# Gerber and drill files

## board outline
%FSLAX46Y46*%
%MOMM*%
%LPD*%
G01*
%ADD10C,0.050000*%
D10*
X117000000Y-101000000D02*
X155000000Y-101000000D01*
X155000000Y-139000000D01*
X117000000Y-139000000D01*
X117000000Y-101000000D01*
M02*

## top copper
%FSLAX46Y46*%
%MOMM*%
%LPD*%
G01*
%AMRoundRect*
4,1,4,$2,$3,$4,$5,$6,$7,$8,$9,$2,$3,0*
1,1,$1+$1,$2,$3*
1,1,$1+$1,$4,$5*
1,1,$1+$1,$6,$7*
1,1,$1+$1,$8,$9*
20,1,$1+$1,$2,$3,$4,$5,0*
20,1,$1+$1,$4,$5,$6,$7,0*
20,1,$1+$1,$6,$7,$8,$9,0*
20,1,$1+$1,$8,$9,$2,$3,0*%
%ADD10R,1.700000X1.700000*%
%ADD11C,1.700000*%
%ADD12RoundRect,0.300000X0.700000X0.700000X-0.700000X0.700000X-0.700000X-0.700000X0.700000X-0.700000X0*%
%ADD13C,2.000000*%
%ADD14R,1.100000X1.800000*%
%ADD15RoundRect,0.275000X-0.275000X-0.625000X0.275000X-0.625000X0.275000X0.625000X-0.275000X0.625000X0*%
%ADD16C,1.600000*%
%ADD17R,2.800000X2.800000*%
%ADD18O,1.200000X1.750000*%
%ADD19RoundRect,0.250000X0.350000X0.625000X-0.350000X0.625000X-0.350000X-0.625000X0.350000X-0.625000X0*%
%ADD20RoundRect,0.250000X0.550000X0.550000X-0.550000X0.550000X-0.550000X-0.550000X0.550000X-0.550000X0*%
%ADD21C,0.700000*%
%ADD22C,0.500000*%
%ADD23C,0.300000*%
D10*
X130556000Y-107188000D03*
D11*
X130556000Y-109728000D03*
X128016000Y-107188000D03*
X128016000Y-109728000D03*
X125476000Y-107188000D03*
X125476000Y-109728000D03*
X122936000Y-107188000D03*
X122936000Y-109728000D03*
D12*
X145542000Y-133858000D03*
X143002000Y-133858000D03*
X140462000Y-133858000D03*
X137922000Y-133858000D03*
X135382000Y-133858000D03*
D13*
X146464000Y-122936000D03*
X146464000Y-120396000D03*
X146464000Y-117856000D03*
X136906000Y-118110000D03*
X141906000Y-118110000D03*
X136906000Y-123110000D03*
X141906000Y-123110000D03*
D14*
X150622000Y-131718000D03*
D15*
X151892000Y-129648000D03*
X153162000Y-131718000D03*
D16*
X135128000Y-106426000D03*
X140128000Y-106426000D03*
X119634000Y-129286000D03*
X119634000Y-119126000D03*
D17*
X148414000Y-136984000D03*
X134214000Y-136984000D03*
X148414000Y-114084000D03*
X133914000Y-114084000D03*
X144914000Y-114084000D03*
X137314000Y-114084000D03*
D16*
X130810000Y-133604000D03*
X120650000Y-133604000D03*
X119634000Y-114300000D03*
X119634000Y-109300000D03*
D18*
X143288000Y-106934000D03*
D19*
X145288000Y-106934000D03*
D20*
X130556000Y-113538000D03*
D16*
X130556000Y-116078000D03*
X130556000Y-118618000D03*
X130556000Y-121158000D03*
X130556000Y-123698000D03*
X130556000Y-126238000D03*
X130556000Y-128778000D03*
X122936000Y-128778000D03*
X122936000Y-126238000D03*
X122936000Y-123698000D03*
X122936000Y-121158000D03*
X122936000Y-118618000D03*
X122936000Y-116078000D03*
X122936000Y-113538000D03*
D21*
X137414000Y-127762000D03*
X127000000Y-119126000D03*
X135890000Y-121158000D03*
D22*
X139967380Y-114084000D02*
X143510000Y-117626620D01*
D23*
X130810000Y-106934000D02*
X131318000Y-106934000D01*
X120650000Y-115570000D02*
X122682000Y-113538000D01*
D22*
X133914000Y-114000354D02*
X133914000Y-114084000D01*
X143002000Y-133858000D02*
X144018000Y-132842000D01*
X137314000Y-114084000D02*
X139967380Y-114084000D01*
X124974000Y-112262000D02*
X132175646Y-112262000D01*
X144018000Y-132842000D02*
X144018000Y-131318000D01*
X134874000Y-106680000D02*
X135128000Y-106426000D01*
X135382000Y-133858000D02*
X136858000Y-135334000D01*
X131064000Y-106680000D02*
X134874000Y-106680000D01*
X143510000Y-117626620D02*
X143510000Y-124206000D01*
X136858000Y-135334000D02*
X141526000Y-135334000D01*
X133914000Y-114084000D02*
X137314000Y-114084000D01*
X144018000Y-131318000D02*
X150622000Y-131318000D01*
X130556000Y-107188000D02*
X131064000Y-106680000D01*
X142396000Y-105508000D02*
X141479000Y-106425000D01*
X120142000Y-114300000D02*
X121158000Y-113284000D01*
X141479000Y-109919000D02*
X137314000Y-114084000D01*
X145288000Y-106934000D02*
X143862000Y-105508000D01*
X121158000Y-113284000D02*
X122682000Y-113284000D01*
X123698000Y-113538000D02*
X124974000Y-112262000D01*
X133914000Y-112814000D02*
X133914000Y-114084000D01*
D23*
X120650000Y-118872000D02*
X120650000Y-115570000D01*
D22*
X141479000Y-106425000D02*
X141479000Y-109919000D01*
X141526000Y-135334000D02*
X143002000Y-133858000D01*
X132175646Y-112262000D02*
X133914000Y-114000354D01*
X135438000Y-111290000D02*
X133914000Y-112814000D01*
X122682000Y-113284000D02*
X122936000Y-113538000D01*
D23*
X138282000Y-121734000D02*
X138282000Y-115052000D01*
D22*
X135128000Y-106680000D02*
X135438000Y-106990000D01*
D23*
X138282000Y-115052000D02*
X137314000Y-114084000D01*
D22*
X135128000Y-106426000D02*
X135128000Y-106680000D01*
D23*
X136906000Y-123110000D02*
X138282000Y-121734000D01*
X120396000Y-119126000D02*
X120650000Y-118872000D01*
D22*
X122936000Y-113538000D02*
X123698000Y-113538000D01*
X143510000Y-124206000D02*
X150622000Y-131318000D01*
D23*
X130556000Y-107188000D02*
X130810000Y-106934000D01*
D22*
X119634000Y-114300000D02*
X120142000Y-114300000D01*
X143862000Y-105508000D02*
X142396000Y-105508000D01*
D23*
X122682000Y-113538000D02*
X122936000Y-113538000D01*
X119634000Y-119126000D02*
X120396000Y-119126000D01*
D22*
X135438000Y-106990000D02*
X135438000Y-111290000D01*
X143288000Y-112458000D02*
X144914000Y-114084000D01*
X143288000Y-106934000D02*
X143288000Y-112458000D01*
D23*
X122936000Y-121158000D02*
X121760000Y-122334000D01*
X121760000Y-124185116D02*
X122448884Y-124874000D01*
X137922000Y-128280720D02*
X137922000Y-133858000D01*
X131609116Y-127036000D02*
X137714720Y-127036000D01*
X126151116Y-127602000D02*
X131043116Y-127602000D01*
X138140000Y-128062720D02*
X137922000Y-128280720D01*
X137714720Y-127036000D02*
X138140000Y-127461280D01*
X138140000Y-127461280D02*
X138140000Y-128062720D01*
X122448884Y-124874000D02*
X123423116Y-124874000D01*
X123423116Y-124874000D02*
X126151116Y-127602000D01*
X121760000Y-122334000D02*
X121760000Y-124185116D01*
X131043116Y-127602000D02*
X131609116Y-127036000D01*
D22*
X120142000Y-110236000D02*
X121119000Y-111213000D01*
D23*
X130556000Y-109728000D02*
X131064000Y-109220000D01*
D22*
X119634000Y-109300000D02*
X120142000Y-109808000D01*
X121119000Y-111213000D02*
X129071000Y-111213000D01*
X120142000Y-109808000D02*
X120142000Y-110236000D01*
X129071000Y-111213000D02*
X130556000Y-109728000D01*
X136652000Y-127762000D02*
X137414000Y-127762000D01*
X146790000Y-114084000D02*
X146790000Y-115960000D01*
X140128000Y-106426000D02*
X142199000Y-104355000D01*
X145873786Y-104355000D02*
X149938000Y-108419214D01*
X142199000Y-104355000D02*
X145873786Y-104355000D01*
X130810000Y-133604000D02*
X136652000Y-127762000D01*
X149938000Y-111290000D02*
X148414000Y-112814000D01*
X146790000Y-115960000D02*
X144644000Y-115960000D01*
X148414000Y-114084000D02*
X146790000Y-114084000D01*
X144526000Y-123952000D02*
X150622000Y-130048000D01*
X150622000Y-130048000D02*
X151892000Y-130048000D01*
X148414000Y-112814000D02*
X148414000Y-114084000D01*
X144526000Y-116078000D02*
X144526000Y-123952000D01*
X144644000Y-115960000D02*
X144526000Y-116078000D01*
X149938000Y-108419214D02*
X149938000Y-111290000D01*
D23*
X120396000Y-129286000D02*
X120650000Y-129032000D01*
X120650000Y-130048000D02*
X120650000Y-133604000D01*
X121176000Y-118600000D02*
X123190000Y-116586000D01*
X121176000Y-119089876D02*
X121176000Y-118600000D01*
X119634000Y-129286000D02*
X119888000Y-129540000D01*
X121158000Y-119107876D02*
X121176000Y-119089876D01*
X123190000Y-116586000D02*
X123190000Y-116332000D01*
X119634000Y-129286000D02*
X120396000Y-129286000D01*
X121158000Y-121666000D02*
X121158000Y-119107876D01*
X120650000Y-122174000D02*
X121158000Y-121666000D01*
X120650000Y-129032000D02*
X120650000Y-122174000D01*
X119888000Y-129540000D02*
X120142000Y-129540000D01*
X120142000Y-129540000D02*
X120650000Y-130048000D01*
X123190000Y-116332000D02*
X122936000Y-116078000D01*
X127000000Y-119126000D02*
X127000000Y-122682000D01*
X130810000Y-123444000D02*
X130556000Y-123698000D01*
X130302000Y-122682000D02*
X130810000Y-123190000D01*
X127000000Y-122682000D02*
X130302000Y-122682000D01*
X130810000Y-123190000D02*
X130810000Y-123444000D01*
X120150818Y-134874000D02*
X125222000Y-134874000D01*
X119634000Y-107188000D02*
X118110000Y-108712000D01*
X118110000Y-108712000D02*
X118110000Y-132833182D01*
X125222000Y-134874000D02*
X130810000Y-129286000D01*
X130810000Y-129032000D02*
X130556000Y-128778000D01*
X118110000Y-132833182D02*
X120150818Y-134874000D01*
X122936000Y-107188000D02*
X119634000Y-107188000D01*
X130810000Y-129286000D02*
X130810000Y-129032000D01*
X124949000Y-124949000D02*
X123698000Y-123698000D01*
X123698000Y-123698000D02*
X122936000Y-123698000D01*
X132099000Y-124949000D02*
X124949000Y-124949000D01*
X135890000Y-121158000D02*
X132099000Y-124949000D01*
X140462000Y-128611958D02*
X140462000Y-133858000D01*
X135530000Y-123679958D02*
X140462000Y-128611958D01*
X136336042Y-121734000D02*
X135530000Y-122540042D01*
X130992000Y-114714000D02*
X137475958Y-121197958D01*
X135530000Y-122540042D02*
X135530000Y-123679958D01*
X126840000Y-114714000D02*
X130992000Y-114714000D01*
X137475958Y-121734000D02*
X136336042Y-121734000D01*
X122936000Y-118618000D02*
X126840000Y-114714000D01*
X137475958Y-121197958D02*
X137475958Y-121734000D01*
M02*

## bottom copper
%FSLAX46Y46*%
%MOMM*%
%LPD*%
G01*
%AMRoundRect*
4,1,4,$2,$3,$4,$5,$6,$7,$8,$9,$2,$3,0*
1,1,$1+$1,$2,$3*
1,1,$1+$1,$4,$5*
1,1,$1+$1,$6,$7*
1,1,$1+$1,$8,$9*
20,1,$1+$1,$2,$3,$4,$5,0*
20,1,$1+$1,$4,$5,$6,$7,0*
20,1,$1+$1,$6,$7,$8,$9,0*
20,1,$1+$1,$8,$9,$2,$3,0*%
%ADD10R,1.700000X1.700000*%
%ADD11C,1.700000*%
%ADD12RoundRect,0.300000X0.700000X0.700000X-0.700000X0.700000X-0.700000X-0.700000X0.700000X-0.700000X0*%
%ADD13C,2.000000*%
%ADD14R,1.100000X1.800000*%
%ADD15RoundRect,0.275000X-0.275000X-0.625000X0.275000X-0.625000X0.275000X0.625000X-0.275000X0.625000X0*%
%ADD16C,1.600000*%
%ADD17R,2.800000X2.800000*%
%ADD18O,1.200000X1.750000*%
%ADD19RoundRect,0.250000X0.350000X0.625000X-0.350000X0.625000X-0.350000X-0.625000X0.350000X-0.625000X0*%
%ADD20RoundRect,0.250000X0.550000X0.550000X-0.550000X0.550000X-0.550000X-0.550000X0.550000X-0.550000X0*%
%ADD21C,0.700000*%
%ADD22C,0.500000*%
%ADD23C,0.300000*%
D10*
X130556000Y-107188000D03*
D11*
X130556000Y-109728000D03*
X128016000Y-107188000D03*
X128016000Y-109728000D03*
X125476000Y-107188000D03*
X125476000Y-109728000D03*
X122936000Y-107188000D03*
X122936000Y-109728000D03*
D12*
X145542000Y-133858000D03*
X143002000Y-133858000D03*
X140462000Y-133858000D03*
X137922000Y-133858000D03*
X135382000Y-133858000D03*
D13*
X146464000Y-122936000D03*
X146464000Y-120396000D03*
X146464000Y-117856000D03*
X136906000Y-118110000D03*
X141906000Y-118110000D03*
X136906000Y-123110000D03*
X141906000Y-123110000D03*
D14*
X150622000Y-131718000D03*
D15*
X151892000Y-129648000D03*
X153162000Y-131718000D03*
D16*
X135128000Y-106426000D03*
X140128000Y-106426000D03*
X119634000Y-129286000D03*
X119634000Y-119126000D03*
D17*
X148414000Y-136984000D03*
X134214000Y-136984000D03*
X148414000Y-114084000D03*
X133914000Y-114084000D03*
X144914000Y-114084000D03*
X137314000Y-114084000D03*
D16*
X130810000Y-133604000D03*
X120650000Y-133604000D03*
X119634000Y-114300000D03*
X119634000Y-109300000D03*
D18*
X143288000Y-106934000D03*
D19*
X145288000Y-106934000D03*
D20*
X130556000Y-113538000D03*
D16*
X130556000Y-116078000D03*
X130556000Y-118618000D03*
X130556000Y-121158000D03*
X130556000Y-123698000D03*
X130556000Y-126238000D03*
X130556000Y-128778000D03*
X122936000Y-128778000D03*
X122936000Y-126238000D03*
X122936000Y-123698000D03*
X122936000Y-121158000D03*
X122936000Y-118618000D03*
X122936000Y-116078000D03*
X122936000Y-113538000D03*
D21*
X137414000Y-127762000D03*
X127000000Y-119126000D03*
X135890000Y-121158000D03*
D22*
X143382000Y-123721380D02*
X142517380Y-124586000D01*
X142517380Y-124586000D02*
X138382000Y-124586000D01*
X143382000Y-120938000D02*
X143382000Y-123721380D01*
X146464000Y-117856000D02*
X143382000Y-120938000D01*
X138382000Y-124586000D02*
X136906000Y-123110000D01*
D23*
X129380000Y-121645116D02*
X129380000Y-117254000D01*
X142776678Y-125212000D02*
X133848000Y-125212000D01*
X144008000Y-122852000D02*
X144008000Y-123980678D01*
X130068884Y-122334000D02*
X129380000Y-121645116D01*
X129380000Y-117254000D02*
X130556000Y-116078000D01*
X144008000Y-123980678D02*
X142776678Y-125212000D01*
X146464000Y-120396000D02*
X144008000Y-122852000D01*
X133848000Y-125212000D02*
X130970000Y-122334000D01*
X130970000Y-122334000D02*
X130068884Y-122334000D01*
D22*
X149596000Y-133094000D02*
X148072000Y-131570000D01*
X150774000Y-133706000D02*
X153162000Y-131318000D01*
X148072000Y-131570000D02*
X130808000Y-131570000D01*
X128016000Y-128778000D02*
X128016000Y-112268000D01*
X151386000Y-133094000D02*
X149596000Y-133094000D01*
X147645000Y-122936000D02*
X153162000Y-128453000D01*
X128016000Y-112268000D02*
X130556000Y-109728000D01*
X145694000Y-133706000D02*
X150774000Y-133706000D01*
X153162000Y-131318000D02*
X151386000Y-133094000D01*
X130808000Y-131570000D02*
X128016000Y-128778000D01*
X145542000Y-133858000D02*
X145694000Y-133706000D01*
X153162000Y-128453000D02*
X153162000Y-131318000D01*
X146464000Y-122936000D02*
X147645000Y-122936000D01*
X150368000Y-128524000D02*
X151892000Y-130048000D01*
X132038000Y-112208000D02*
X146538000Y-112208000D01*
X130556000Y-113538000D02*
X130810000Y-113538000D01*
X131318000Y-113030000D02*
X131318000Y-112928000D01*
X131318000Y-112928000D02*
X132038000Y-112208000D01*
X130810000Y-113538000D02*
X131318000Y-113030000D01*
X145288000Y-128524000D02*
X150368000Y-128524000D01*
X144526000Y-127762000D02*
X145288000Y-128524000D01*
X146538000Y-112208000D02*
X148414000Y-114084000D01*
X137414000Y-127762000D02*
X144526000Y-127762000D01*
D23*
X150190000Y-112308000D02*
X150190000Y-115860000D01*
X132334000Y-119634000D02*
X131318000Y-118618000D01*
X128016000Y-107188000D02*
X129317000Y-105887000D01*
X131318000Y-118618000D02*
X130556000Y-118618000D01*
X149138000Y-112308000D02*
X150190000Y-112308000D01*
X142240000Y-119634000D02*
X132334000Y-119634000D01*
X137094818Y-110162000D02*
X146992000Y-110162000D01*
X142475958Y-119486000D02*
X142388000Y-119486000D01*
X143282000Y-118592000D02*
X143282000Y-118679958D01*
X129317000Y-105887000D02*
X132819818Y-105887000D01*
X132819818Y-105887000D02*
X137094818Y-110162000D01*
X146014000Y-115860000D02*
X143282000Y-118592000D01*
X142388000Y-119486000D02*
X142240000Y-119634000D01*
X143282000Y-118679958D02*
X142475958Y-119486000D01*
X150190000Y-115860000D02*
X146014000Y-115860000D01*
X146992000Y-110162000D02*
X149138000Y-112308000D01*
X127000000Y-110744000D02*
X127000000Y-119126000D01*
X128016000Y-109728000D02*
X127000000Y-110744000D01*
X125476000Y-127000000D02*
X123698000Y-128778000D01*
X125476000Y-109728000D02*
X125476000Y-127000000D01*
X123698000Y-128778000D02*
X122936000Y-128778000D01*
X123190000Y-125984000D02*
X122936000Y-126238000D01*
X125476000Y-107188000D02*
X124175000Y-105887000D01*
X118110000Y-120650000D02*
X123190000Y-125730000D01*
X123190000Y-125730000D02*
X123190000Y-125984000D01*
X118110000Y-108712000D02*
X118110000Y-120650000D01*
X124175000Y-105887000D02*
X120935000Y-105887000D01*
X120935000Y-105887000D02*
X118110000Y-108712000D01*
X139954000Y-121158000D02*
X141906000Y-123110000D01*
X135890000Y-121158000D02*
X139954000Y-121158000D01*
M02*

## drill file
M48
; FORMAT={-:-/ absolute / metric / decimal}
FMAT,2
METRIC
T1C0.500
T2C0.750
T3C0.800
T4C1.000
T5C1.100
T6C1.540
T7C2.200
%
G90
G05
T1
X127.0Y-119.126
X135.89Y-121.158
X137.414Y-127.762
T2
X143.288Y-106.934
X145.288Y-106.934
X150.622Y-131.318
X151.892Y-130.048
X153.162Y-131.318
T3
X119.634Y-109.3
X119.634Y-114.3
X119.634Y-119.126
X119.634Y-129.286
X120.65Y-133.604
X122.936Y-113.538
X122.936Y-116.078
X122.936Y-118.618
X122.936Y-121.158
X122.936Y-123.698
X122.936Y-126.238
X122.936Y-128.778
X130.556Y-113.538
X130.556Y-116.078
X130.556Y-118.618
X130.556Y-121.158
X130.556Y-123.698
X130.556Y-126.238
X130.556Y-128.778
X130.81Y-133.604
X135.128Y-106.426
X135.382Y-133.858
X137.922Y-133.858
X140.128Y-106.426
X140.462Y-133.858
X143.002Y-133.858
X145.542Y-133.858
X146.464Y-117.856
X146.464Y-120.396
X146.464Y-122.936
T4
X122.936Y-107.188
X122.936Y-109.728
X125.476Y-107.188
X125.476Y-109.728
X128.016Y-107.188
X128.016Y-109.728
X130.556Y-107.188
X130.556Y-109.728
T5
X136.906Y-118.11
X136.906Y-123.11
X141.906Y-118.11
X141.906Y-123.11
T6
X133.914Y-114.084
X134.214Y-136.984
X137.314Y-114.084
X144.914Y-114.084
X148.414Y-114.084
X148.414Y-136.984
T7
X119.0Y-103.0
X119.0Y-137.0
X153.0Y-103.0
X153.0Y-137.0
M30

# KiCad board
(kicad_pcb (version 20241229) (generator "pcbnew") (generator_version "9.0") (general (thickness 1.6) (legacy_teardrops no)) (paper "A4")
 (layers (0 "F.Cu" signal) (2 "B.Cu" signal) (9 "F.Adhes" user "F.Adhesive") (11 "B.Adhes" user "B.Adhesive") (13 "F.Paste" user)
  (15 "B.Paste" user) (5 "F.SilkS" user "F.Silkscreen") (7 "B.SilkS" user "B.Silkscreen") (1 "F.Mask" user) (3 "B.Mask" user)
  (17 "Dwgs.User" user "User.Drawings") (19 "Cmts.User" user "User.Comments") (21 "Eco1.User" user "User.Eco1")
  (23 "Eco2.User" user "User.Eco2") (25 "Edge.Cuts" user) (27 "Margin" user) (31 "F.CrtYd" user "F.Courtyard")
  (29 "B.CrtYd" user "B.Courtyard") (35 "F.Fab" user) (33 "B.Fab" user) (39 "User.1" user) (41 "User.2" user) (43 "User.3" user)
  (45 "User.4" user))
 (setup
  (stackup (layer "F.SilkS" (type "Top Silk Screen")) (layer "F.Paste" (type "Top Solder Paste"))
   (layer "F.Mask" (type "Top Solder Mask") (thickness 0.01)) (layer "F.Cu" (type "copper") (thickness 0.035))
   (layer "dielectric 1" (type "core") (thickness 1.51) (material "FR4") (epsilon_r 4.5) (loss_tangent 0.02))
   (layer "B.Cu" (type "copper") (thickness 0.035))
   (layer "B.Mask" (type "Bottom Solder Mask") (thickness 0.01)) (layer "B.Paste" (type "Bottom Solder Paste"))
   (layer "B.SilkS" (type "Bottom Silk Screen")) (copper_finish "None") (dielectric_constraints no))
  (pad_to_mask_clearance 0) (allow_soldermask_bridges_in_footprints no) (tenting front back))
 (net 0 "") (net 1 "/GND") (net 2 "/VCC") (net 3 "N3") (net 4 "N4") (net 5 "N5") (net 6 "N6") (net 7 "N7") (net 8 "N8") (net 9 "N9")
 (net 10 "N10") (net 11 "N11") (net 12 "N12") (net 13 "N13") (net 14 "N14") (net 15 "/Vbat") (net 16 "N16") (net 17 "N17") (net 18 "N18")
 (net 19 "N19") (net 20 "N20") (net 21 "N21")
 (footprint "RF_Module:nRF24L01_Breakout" (layer "F.Cu") (at 130.556 107.188 -90)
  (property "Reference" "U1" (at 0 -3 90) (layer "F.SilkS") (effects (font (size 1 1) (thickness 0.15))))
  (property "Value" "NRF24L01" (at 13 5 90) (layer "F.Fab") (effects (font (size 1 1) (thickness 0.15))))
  (pad "1" thru_hole rect (at 0 0 270) (size 1.7 1.7) (drill 1) (layers "*.Cu" "*.Mask") (remove_unused_layers no) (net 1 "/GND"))
  (pad "2" thru_hole circle (at 2.54 0 270) (size 1.7 1.7) (drill 1) (layers "*.Cu" "*.Mask") (remove_unused_layers no) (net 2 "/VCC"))
  (pad "3" thru_hole circle (at 0 2.54 270) (size 1.7 1.7) (drill 1) (layers "*.Cu" "*.Mask") (remove_unused_layers no) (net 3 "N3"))
  (pad "4" thru_hole circle (at 2.54 2.54 270) (size 1.7 1.7) (drill 1) (layers "*.Cu" "*.Mask") (remove_unused_layers no) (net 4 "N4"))
  (pad "5" thru_hole circle (at 0 5.08 270) (size 1.7 1.7) (drill 1) (layers "*.Cu" "*.Mask") (remove_unused_layers no) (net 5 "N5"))
  (pad "6" thru_hole circle (at 2.54 5.08 270) (size 1.7 1.7) (drill 1) (layers "*.Cu" "*.Mask") (remove_unused_layers no) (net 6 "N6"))
  (pad "7" thru_hole circle (at 0 7.62 270) (size 1.7 1.7) (drill 1) (layers "*.Cu" "*.Mask") (remove_unused_layers no) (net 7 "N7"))
  (pad "8" thru_hole circle (at 2.54 7.62 270) (size 1.7 1.7) (drill 1) (layers "*.Cu" "*.Mask") (remove_unused_layers no) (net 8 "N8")))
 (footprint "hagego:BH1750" (layer "F.Cu") (at 140.462 135.128 180)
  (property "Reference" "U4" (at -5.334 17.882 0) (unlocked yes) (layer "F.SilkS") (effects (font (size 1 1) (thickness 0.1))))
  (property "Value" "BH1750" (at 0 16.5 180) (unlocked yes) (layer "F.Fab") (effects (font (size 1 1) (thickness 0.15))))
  (pad "1" thru_hole roundrect (at -5.08 1.27 180) (size 2 2) (drill 0.8) (layers "*.Cu" "*.Mask") (remove_unused_layers no)
   (roundrect_rratio 0.15) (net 2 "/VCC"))
  (pad "2" thru_hole roundrect (at -2.54 1.27 180) (size 2 2) (drill 0.8) (layers "*.Cu" "*.Mask") (remove_unused_layers no)
   (roundrect_rratio 0.15) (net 1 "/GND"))
  (pad "3" thru_hole roundrect (at 0 1.27 180) (size 2 2) (drill 0.8) (layers "*.Cu" "*.Mask") (remove_unused_layers no)
   (roundrect_rratio 0.15) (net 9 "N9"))
  (pad "4" thru_hole roundrect (at 2.54 1.27 180) (size 2 2) (drill 0.8) (layers "*.Cu" "*.Mask") (remove_unused_layers no)
   (roundrect_rratio 0.15) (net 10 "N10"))
  (pad "5" thru_hole roundrect (at 5.08 1.27 180) (size 2 2) (drill 0.8) (layers "*.Cu" "*.Mask") (remove_unused_layers no)
   (roundrect_rratio 0.15) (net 1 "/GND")))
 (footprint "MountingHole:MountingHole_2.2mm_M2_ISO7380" (layer "F.Cu") (at 153 137)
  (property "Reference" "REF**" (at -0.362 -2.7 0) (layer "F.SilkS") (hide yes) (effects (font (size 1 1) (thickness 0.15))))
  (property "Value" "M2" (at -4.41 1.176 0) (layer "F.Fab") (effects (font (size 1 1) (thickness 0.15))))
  (pad "" np_thru_hole circle (at 0 0) (size 2.2 2.2) (drill 2.2) (layers "*.Cu" "*.Mask")))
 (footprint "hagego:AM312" (layer "F.Cu") (at 148.336 120.396 90)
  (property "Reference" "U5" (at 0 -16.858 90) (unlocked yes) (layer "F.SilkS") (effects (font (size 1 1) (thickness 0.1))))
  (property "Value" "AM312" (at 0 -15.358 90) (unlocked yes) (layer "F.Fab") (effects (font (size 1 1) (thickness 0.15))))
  (pad "1" thru_hole circle (at -2.54 -1.872 90) (size 2 2) (drill 0.8) (layers "*.Cu" "*.Mask") (remove_unused_layers no) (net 2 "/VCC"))
  (pad "2" thru_hole circle (at 0 -1.872 90) (size 2 2) (drill 0.8) (layers "*.Cu" "*.Mask") (remove_unused_layers no) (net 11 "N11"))
  (pad "3" thru_hole circle (at 2.54 -1.872 90) (size 2 2) (drill 0.8) (layers "*.Cu" "*.Mask") (remove_unused_layers no) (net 1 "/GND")))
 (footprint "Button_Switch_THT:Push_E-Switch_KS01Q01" (layer "F.Cu") (at 136.906 118.11)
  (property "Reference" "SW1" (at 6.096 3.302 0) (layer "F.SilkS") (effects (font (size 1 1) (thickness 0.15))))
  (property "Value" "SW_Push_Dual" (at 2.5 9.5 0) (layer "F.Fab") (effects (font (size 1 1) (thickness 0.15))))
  (pad "1" thru_hole circle (at 0 0) (size 2 2) (drill 1.1) (layers "*.Cu" "*.Mask") (remove_unused_layers no) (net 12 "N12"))
  (pad "2" thru_hole circle (at 5 0) (size 2 2) (drill 1.1) (layers "*.Cu" "*.Mask") (remove_unused_layers no) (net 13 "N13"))
  (pad "3" thru_hole circle (at 0 5) (size 2 2) (drill 1.1) (layers "*.Cu" "*.Mask") (remove_unused_layers no) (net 1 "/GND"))
  (pad "4" thru_hole circle (at 5 5) (size 2 2) (drill 1.1) (layers "*.Cu" "*.Mask") (remove_unused_layers no) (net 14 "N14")))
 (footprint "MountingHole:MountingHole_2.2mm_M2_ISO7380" (layer "F.Cu") (at 119 137)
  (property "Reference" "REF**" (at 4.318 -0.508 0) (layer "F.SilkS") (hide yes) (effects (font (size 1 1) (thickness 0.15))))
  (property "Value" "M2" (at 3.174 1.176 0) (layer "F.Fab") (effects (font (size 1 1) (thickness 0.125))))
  (pad "" np_thru_hole circle (at 0 0) (size 2.2 2.2) (drill 2.2) (layers "*.Cu" "*.Mask")))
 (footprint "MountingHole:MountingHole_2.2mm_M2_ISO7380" (layer "F.Cu") (at 119 103)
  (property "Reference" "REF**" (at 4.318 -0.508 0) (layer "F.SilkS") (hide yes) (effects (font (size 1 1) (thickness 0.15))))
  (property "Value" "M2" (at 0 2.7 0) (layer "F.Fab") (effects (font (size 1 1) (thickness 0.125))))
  (pad "" np_thru_hole circle (at 0 0) (size 2.2 2.2) (drill 2.2) (layers "*.Cu" "*.Mask")))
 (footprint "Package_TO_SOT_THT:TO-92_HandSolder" (layer "F.Cu") (at 150.622 131.318)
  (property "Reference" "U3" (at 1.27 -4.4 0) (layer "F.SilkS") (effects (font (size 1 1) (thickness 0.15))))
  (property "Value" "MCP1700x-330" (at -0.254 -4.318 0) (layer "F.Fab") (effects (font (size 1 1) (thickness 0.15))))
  (pad "1" thru_hole rect (at 0 0) (size 1.1 1.8) (drill 0.75 (offset 0 0.4)) (layers "*.Cu" "*.Mask") (remove_unused_layers no)
   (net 1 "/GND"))
  (pad "2" thru_hole roundrect (at 1.27 -1.27) (size 1.1 1.8) (drill 0.75 (offset 0 -0.4)) (layers "*.Cu" "*.Mask")
   (remove_unused_layers no) (roundrect_rratio 0.25) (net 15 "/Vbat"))
  (pad "3" thru_hole roundrect (at 2.54 0) (size 1.1 1.8) (drill 0.75 (offset 0 0.4)) (layers "*.Cu" "*.Mask") (remove_unused_layers no)
   (roundrect_rratio 0.25) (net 2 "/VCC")))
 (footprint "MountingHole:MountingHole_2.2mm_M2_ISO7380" (layer "F.Cu") (at 153 103)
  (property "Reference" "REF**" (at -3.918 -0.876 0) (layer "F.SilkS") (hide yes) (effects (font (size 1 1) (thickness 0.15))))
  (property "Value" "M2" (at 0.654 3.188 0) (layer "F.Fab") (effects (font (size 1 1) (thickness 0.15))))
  (pad "" np_thru_hole circle (at 0 0) (size 2.2 2.2) (drill 2.2) (layers "*.Cu" "*.Mask")))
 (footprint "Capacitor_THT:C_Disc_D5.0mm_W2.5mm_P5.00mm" (layer "F.Cu") (at 135.128 106.426)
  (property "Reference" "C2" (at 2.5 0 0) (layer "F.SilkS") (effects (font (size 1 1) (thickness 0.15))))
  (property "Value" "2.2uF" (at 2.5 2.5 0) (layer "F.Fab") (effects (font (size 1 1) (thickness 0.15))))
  (pad "1" thru_hole circle (at 0 0) (size 1.6 1.6) (drill 0.8) (layers "*.Cu" "*.Mask") (remove_unused_layers no) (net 1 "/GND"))
  (pad "2" thru_hole circle (at 5 0) (size 1.6 1.6) (drill 0.8) (layers "*.Cu" "*.Mask") (remove_unused_layers no) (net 15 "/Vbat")))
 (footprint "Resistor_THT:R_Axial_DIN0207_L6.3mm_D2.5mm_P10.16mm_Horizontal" (layer "B.Cu") (at 119.634 129.286 90)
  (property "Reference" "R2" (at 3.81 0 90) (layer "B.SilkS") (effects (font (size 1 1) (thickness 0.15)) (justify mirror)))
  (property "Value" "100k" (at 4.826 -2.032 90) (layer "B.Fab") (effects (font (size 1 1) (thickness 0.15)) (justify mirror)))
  (pad "1" thru_hole circle (at 0 0 90) (size 1.6 1.6) (drill 0.8) (layers "*.Cu" "*.Mask") (remove_unused_layers no) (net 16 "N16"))
  (pad "2" thru_hole circle (at 10.16 0 90) (size 1.6 1.6) (drill 0.8) (layers "*.Cu" "*.Mask") (remove_unused_layers no) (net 1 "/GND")))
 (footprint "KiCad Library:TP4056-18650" (layer "B.Cu") (at 150.114 138.684 90)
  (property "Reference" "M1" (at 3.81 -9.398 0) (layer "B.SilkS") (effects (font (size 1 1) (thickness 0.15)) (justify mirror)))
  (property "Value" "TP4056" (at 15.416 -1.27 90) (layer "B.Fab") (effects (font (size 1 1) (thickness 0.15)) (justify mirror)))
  (pad "1" thru_hole rect (at 1.7 -1.7 90) (size 2.8 2.8) (drill 1.54) (layers "*.Cu" "*.Mask") (remove_unused_layers no) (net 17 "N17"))
  (pad "2" thru_hole rect (at 1.7 -15.9 90) (size 2.8 2.8) (drill 1.54) (layers "*.Cu" "*.Mask") (remove_unused_layers no) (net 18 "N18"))
  (pad "3" thru_hole rect (at 24.6 -1.7 90) (size 2.8 2.8) (drill 1.54) (layers "*.Cu" "*.Mask") (remove_unused_layers no) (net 15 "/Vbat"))
  (pad "4" thru_hole rect (at 24.6 -16.2 90) (size 2.8 2.8) (drill 1.54) (layers "*.Cu" "*.Mask") (remove_unused_layers no) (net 1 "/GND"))
  (pad "5" thru_hole rect (at 24.6 -5.2 90) (size 2.8 2.8) (drill 1.54) (layers "*.Cu" "*.Mask") (remove_unused_layers no) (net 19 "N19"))
  (pad "6" thru_hole rect (at 24.6 -12.8 90) (size 2.8 2.8) (drill 1.54) (layers "*.Cu" "*.Mask") (remove_unused_layers no) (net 1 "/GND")))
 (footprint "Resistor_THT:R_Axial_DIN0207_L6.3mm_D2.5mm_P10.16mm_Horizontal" (layer "B.Cu") (at 130.81 133.604 180)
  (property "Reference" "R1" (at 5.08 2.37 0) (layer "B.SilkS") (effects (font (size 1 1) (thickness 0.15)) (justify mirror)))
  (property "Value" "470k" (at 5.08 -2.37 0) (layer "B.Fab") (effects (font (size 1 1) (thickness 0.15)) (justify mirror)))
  (pad "1" thru_hole circle (at 0 0 180) (size 1.6 1.6) (drill 0.8) (layers "*.Cu" "*.Mask") (remove_unused_layers no) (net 15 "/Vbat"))
  (pad "2" thru_hole circle (at 10.16 0 180) (size 1.6 1.6) (drill 0.8) (layers "*.Cu" "*.Mask") (remove_unused_layers no) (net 16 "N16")))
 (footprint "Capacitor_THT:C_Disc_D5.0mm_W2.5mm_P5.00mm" (layer "B.Cu") (at 119.634 114.3 90)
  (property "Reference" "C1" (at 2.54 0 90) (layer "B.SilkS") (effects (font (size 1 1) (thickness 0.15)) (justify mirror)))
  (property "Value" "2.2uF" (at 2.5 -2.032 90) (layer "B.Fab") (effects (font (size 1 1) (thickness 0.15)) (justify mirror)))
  (pad "1" thru_hole circle (at 0 0 90) (size 1.6 1.6) (drill 0.8) (layers "*.Cu" "*.Mask") (remove_unused_layers no) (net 1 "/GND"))
  (pad "2" thru_hole circle (at 5 0 90) (size 1.6 1.6) (drill 0.8) (layers "*.Cu" "*.Mask") (remove_unused_layers no) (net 2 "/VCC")))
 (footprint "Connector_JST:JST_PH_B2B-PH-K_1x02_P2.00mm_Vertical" (layer "B.Cu") (at 145.288 106.934 180)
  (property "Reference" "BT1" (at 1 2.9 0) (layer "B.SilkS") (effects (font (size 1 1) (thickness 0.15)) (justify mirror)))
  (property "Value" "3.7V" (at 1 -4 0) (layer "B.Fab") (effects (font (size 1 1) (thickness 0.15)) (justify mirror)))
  (pad "1" thru_hole oval (at 2 0 180) (size 1.2 1.75) (drill 0.75) (layers "*.Cu" "*.Mask") (remove_unused_layers no) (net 19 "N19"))
  (pad "2" thru_hole roundrect (at 0 0 180) (size 1.2 1.75) (drill 0.75) (layers "*.Cu" "*.Mask") (remove_unused_layers no)
   (roundrect_rratio 0.208333) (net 1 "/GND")))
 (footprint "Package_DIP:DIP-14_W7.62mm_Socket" (layer "B.Cu") (at 130.556 113.538 180)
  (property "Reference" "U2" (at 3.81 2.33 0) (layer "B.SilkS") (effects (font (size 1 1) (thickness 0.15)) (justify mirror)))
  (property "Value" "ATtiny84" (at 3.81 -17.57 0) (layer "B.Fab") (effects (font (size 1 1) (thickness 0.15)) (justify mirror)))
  (pad "1" thru_hole roundrect (at 0 0 180) (size 1.6 1.6) (drill 0.8) (layers "*.Cu" "*.Mask") (remove_unused_layers no)
   (roundrect_rratio 0.15625) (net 15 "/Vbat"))
  (pad "2" thru_hole circle (at 0 -2.54 180) (size 1.6 1.6) (drill 0.8) (layers "*.Cu" "*.Mask") (remove_unused_layers no) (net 11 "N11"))
  (pad "3" thru_hole circle (at 0 -5.08 180) (size 1.6 1.6) (drill 0.8) (layers "*.Cu" "*.Mask") (remove_unused_layers no) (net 3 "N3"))
  (pad "4" thru_hole circle (at 0 -7.62 180) (size 1.6 1.6) (drill 0.8) (layers "*.Cu" "*.Mask") (remove_unused_layers no) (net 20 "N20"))
  (pad "5" thru_hole circle (at 0 -10.16 180) (size 1.6 1.6) (drill 0.8) (layers "*.Cu" "*.Mask") (remove_unused_layers no) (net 4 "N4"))
  (pad "6" thru_hole circle (at 0 -12.7 180) (size 1.6 1.6) (drill 0.8) (layers "*.Cu" "*.Mask") (remove_unused_layers no) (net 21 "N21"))
  (pad "7" thru_hole circle (at 0 -15.24 180) (size 1.6 1.6) (drill 0.8) (layers "*.Cu" "*.Mask") (remove_unused_layers no) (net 7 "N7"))
  (pad "8" thru_hole circle (at 7.62 -15.24 180) (size 1.6 1.6) (drill 0.8) (layers "*.Cu" "*.Mask") (remove_unused_layers no) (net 6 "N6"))
  (pad "9" thru_hole circle (at 7.62 -12.7 180) (size 1.6 1.6) (drill 0.8) (layers "*.Cu" "*.Mask") (remove_unused_layers no) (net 5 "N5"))
  (pad "10" thru_hole circle (at 7.62 -10.16 180) (size 1.6 1.6) (drill 0.8) (layers "*.Cu" "*.Mask") (remove_unused_layers no)
   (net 14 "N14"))
  (pad "11" thru_hole circle (at 7.62 -7.62 180) (size 1.6 1.6) (drill 0.8) (layers "*.Cu" "*.Mask") (remove_unused_layers no)
   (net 10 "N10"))
  (pad "12" thru_hole circle (at 7.62 -5.08 180) (size 1.6 1.6) (drill 0.8) (layers "*.Cu" "*.Mask") (remove_unused_layers no) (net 9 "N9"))
  (pad "13" thru_hole circle (at 7.62 -2.54 180) (size 1.6 1.6) (drill 0.8) (layers "*.Cu" "*.Mask") (remove_unused_layers no)
   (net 16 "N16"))
  (pad "14" thru_hole circle (at 7.62 0 180) (size 1.6 1.6) (drill 0.8) (layers "*.Cu" "*.Mask") (remove_unused_layers no) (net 1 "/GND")))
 (gr_rect (start 117 101) (end 155 139) (stroke (width 0.05) (type solid)) (fill no) (layer "Edge.Cuts"))
 (segment (start 139.96738 114.084) (end 143.51 117.62662) (width 0.5) (layer "F.Cu") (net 1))
 (segment (start 130.81 106.934) (end 131.318 106.934) (width 0.3) (layer "F.Cu") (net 1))
 (segment (start 120.65 115.57) (end 122.682 113.538) (width 0.3) (layer "F.Cu") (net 1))
 (segment (start 133.914 114.000354) (end 133.914 114.084) (width 0.5) (layer "F.Cu") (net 1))
 (segment (start 143.002 133.858) (end 144.018 132.842) (width 0.5) (layer "F.Cu") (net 1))
 (segment (start 137.314 114.084) (end 139.96738 114.084) (width 0.5) (layer "F.Cu") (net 1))
 (segment (start 124.974 112.262) (end 132.175646 112.262) (width 0.5) (layer "F.Cu") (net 1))
 (segment (start 144.018 132.842) (end 144.018 131.318) (width 0.5) (layer "F.Cu") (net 1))
 (segment (start 134.874 106.68) (end 135.128 106.426) (width 0.5) (layer "F.Cu") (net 1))
 (segment (start 135.382 133.858) (end 136.858 135.334) (width 0.5) (layer "F.Cu") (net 1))
 (segment (start 131.064 106.68) (end 134.874 106.68) (width 0.5) (layer "F.Cu") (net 1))
 (segment (start 143.51 117.62662) (end 143.51 124.206) (width 0.5) (layer "F.Cu") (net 1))
 (segment (start 136.858 135.334) (end 141.526 135.334) (width 0.5) (layer "F.Cu") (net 1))
 (segment (start 133.914 114.084) (end 137.314 114.084) (width 0.5) (layer "F.Cu") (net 1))
 (segment (start 144.018 131.318) (end 150.622 131.318) (width 0.5) (layer "F.Cu") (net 1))
 (segment (start 130.556 107.188) (end 131.064 106.68) (width 0.5) (layer "F.Cu") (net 1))
 (segment (start 142.396 105.508) (end 141.479 106.425) (width 0.5) (layer "F.Cu") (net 1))
 (segment (start 120.142 114.3) (end 121.158 113.284) (width 0.5) (layer "F.Cu") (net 1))
 (segment (start 141.479 109.919) (end 137.314 114.084) (width 0.5) (layer "F.Cu") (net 1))
 (segment (start 145.288 106.934) (end 143.862 105.508) (width 0.5) (layer "F.Cu") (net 1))
 (segment (start 121.158 113.284) (end 122.682 113.284) (width 0.5) (layer "F.Cu") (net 1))
 (segment (start 123.698 113.538) (end 124.974 112.262) (width 0.5) (layer "F.Cu") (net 1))
 (segment (start 133.914 112.814) (end 133.914 114.084) (width 0.5) (layer "F.Cu") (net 1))
 (segment (start 120.65 118.872) (end 120.65 115.57) (width 0.3) (layer "F.Cu") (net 1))
 (segment (start 141.479 106.425) (end 141.479 109.919) (width 0.5) (layer "F.Cu") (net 1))
 (segment (start 141.526 135.334) (end 143.002 133.858) (width 0.5) (layer "F.Cu") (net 1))
 (segment (start 132.175646 112.262) (end 133.914 114.000354) (width 0.5) (layer "F.Cu") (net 1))
 (segment (start 135.438 111.29) (end 133.914 112.814) (width 0.5) (layer "F.Cu") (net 1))
 (segment (start 122.682 113.284) (end 122.936 113.538) (width 0.5) (layer "F.Cu") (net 1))
 (segment (start 138.282 121.734) (end 138.282 115.052) (width 0.3) (layer "F.Cu") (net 1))
 (segment (start 135.128 106.68) (end 135.438 106.99) (width 0.5) (layer "F.Cu") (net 1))
 (segment (start 138.282 115.052) (end 137.314 114.084) (width 0.3) (layer "F.Cu") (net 1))
 (segment (start 135.128 106.426) (end 135.128 106.68) (width 0.5) (layer "F.Cu") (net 1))
 (segment (start 136.906 123.11) (end 138.282 121.734) (width 0.3) (layer "F.Cu") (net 1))
 (segment (start 120.396 119.126) (end 120.65 118.872) (width 0.3) (layer "F.Cu") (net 1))
 (segment (start 122.936 113.538) (end 123.698 113.538) (width 0.5) (layer "F.Cu") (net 1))
 (segment (start 143.51 124.206) (end 150.622 131.318) (width 0.5) (layer "F.Cu") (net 1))
 (segment (start 130.556 107.188) (end 130.81 106.934) (width 0.3) (layer "F.Cu") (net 1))
 (segment (start 119.634 114.3) (end 120.142 114.3) (width 0.5) (layer "F.Cu") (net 1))
 (segment (start 143.862 105.508) (end 142.396 105.508) (width 0.5) (layer "F.Cu") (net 1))
 (segment (start 122.682 113.538) (end 122.936 113.538) (width 0.3) (layer "F.Cu") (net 1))
 (segment (start 119.634 119.126) (end 120.396 119.126) (width 0.3) (layer "F.Cu") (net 1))
 (segment (start 135.438 106.99) (end 135.438 111.29) (width 0.5) (layer "F.Cu") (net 1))
 (segment (start 143.382 123.72138) (end 142.51738 124.586) (width 0.5) (layer "B.Cu") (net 1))
 (segment (start 142.51738 124.586) (end 138.382 124.586) (width 0.5) (layer "B.Cu") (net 1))
 (segment (start 143.382 120.938) (end 143.382 123.72138) (width 0.5) (layer "B.Cu") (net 1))
 (segment (start 146.464 117.856) (end 143.382 120.938) (width 0.5) (layer "B.Cu") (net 1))
 (segment (start 138.382 124.586) (end 136.906 123.11) (width 0.5) (layer "B.Cu") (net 1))
 (segment (start 143.288 112.458) (end 144.914 114.084) (width 0.5) (layer "F.Cu") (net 19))
 (segment (start 143.288 106.934) (end 143.288 112.458) (width 0.5) (layer "F.Cu") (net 19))
 (segment (start 122.936 121.158) (end 121.76 122.334) (width 0.3) (layer "F.Cu") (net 10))
 (segment (start 121.76 124.185116) (end 122.448884 124.874) (width 0.3) (layer "F.Cu") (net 10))
 (segment (start 137.922 128.28072) (end 137.922 133.858) (width 0.3) (layer "F.Cu") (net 10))
 (segment (start 131.609116 127.036) (end 137.71472 127.036) (width 0.3) (layer "F.Cu") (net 10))
 (segment (start 126.151116 127.602) (end 131.043116 127.602) (width 0.3) (layer "F.Cu") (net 10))
 (segment (start 138.14 128.06272) (end 137.922 128.28072) (width 0.3) (layer "F.Cu") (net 10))
 (segment (start 137.71472 127.036) (end 138.14 127.46128) (width 0.3) (layer "F.Cu") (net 10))
 (segment (start 138.14 127.46128) (end 138.14 128.06272) (width 0.3) (layer "F.Cu") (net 10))
 (segment (start 122.448884 124.874) (end 123.423116 124.874) (width 0.3) (layer "F.Cu") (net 10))
 (segment (start 123.423116 124.874) (end 126.151116 127.602) (width 0.3) (layer "F.Cu") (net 10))
 (segment (start 121.76 122.334) (end 121.76 124.185116) (width 0.3) (layer "F.Cu") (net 10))
 (segment (start 131.043116 127.602) (end 131.609116 127.036) (width 0.3) (layer "F.Cu") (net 10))
 (segment (start 129.38 121.645116) (end 129.38 117.254) (width 0.3) (layer "B.Cu") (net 11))
 (segment (start 142.776678 125.212) (end 133.848 125.212) (width 0.3) (layer "B.Cu") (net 11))
 (segment (start 144.008 122.852) (end 144.008 123.980678) (width 0.3) (layer "B.Cu") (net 11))
 (segment (start 130.068884 122.334) (end 129.38 121.645116) (width 0.3) (layer "B.Cu") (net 11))
 (segment (start 129.38 117.254) (end 130.556 116.078) (width 0.3) (layer "B.Cu") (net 11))
 (segment (start 144.008 123.980678) (end 142.776678 125.212) (width 0.3) (layer "B.Cu") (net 11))
 (segment (start 146.464 120.396) (end 144.008 122.852) (width 0.3) (layer "B.Cu") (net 11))
 (segment (start 133.848 125.212) (end 130.97 122.334) (width 0.3) (layer "B.Cu") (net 11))
 (segment (start 130.97 122.334) (end 130.068884 122.334) (width 0.3) (layer "B.Cu") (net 11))
 (segment (start 120.142 110.236) (end 121.119 111.213) (width 0.5) (layer "F.Cu") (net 2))
 (segment (start 130.556 109.728) (end 131.064 109.22) (width 0.3) (layer "F.Cu") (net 2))
 (segment (start 119.634 109.3) (end 120.142 109.808) (width 0.5) (layer "F.Cu") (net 2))
 (segment (start 121.119 111.213) (end 129.071 111.213) (width 0.5) (layer "F.Cu") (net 2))
 (segment (start 120.142 109.808) (end 120.142 110.236) (width 0.5) (layer "F.Cu") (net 2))
 (segment (start 129.071 111.213) (end 130.556 109.728) (width 0.5) (layer "F.Cu") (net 2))
 (segment (start 149.596 133.094) (end 148.072 131.57) (width 0.5) (layer "B.Cu") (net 2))
 (segment (start 150.774 133.706) (end 153.162 131.318) (width 0.5) (layer "B.Cu") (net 2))
 (segment (start 148.072 131.57) (end 130.808 131.57) (width 0.5) (layer "B.Cu") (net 2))
 (segment (start 128.016 128.778) (end 128.016 112.268) (width 0.5) (layer "B.Cu") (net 2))
 (segment (start 151.386 133.094) (end 149.596 133.094) (width 0.5) (layer "B.Cu") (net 2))
 (segment (start 147.645 122.936) (end 153.162 128.453) (width 0.5) (layer "B.Cu") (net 2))
 (segment (start 128.016 112.268) (end 130.556 109.728) (width 0.5) (layer "B.Cu") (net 2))
 (segment (start 145.694 133.706) (end 150.774 133.706) (width 0.5) (layer "B.Cu") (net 2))
 (segment (start 153.162 131.318) (end 151.386 133.094) (width 0.5) (layer "B.Cu") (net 2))
 (segment (start 130.808 131.57) (end 128.016 128.778) (width 0.5) (layer "B.Cu") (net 2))
 (segment (start 145.542 133.858) (end 145.694 133.706) (width 0.5) (layer "B.Cu") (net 2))
 (segment (start 153.162 128.453) (end 153.162 131.318) (width 0.5) (layer "B.Cu") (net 2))
 (segment (start 146.464 122.936) (end 147.645 122.936) (width 0.5) (layer "B.Cu") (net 2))
 (segment (start 136.652 127.762) (end 137.414 127.762) (width 0.5) (layer "F.Cu") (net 15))
 (segment (start 146.79 114.084) (end 146.79 115.96) (width 0.5) (layer "F.Cu") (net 15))
 (segment (start 140.128 106.426) (end 142.199 104.355) (width 0.5) (layer "F.Cu") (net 15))
 (segment (start 145.873786 104.355) (end 149.938 108.419214) (width 0.5) (layer "F.Cu") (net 15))
 (segment (start 142.199 104.355) (end 145.873786 104.355) (width 0.5) (layer "F.Cu") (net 15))
 (segment (start 130.81 133.604) (end 136.652 127.762) (width 0.5) (layer "F.Cu") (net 15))
 (segment (start 149.938 111.29) (end 148.414 112.814) (width 0.5) (layer "F.Cu") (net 15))
 (segment (start 146.79 115.96) (end 144.644 115.96) (width 0.5) (layer "F.Cu") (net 15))
 (segment (start 148.414 114.084) (end 146.79 114.084) (width 0.5) (layer "F.Cu") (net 15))
 (segment (start 144.526 123.952) (end 150.622 130.048) (width 0.5) (layer "F.Cu") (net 15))
 (segment (start 150.622 130.048) (end 151.892 130.048) (width 0.5) (layer "F.Cu") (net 15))
 (segment (start 148.414 112.814) (end 148.414 114.084) (width 0.5) (layer "F.Cu") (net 15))
 (segment (start 144.526 116.078) (end 144.526 123.952) (width 0.5) (layer "F.Cu") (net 15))
 (segment (start 144.644 115.96) (end 144.526 116.078) (width 0.5) (layer "F.Cu") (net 15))
 (segment (start 149.938 108.419214) (end 149.938 111.29) (width 0.5) (layer "F.Cu") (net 15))
 (via (at 137.414 127.762) (size 0.7) (drill 0.5) (layers "F.Cu" "B.Cu") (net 15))
 (segment (start 150.368 128.524) (end 151.892 130.048) (width 0.5) (layer "B.Cu") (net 15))
 (segment (start 132.038 112.208) (end 146.538 112.208) (width 0.5) (layer "B.Cu") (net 15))
 (segment (start 130.556 113.538) (end 130.81 113.538) (width 0.5) (layer "B.Cu") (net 15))
 (segment (start 131.318 113.03) (end 131.318 112.928) (width 0.5) (layer "B.Cu") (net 15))
 (segment (start 131.318 112.928) (end 132.038 112.208) (width 0.5) (layer "B.Cu") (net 15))
 (segment (start 130.81 113.538) (end 131.318 113.03) (width 0.5) (layer "B.Cu") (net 15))
 (segment (start 145.288 128.524) (end 150.368 128.524) (width 0.5) (layer "B.Cu") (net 15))
 (segment (start 144.526 127.762) (end 145.288 128.524) (width 0.5) (layer "B.Cu") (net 15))
 (segment (start 146.538 112.208) (end 148.414 114.084) (width 0.5) (layer "B.Cu") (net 15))
 (segment (start 137.414 127.762) (end 144.526 127.762) (width 0.5) (layer "B.Cu") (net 15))
 (segment (start 120.396 129.286) (end 120.65 129.032) (width 0.3) (layer "F.Cu") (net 16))
 (segment (start 120.65 130.048) (end 120.65 133.604) (width 0.3) (layer "F.Cu") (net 16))
 (segment (start 121.176 118.6) (end 123.19 116.586) (width 0.3) (layer "F.Cu") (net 16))
 (segment (start 121.176 119.089876) (end 121.176 118.6) (width 0.3) (layer "F.Cu") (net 16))
 (segment (start 119.634 129.286) (end 119.888 129.54) (width 0.3) (layer "F.Cu") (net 16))
 (segment (start 121.158 119.107876) (end 121.176 119.089876) (width 0.3) (layer "F.Cu") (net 16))
 (segment (start 123.19 116.586) (end 123.19 116.332) (width 0.3) (layer "F.Cu") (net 16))
 (segment (start 119.634 129.286) (end 120.396 129.286) (width 0.3) (layer "F.Cu") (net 16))
 (segment (start 121.158 121.666) (end 121.158 119.107876) (width 0.3) (layer "F.Cu") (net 16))
 (segment (start 120.65 122.174) (end 121.158 121.666) (width 0.3) (layer "F.Cu") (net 16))
 (segment (start 120.65 129.032) (end 120.65 122.174) (width 0.3) (layer "F.Cu") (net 16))
 (segment (start 119.888 129.54) (end 120.142 129.54) (width 0.3) (layer "F.Cu") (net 16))
 (segment (start 120.142 129.54) (end 120.65 130.048) (width 0.3) (layer "F.Cu") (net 16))
 (segment (start 123.19 116.332) (end 122.936 116.078) (width 0.3) (layer "F.Cu") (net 16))
 (segment (start 150.19 112.308) (end 150.19 115.86) (width 0.3) (layer "B.Cu") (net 3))
 (segment (start 132.334 119.634) (end 131.318 118.618) (width 0.3) (layer "B.Cu") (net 3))
 (segment (start 128.016 107.188) (end 129.317 105.887) (width 0.3) (layer "B.Cu") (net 3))
 (segment (start 131.318 118.618) (end 130.556 118.618) (width 0.3) (layer "B.Cu") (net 3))
 (segment (start 149.138 112.308) (end 150.19 112.308) (width 0.3) (layer "B.Cu") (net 3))
 (segment (start 142.24 119.634) (end 132.334 119.634) (width 0.3) (layer "B.Cu") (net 3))
 (segment (start 137.094818 110.162) (end 146.992 110.162) (width 0.3) (layer "B.Cu") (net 3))
 (segment (start 142.475958 119.486) (end 142.388 119.486) (width 0.3) (layer "B.Cu") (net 3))
 (segment (start 143.282 118.592) (end 143.282 118.679958) (width 0.3) (layer "B.Cu") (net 3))
 (segment (start 129.317 105.887) (end 132.819818 105.887) (width 0.3) (layer "B.Cu") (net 3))
 (segment (start 132.819818 105.887) (end 137.094818 110.162) (width 0.3) (layer "B.Cu") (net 3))
 (segment (start 146.014 115.86) (end 143.282 118.592) (width 0.3) (layer "B.Cu") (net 3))
 (segment (start 142.388 119.486) (end 142.24 119.634) (width 0.3) (layer "B.Cu") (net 3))
 (segment (start 143.282 118.679958) (end 142.475958 119.486) (width 0.3) (layer "B.Cu") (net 3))
 (segment (start 150.19 115.86) (end 146.014 115.86) (width 0.3) (layer "B.Cu") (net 3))
 (segment (start 146.992 110.162) (end 149.138 112.308) (width 0.3) (layer "B.Cu") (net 3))
 (segment (start 127 119.126) (end 127 122.682) (width 0.3) (layer "F.Cu") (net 4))
 (segment (start 130.81 123.444) (end 130.556 123.698) (width 0.3) (layer "F.Cu") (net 4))
 (segment (start 130.302 122.682) (end 130.81 123.19) (width 0.3) (layer "F.Cu") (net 4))
 (segment (start 127 122.682) (end 130.302 122.682) (width 0.3) (layer "F.Cu") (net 4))
 (segment (start 130.81 123.19) (end 130.81 123.444) (width 0.3) (layer "F.Cu") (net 4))
 (via (at 127 119.126) (size 0.7) (drill 0.5) (layers "F.Cu" "B.Cu") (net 4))
 (segment (start 127 110.744) (end 127 119.126) (width 0.3) (layer "B.Cu") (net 4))
 (segment (start 128.016 109.728) (end 127 110.744) (width 0.3) (layer "B.Cu") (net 4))
 (segment (start 125.476 127) (end 123.698 128.778) (width 0.3) (layer "B.Cu") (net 6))
 (segment (start 125.476 109.728) (end 125.476 127) (width 0.3) (layer "B.Cu") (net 6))
 (segment (start 123.698 128.778) (end 122.936 128.778) (width 0.3) (layer "B.Cu") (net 6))
 (segment (start 123.19 125.984) (end 122.936 126.238) (width 0.3) (layer "B.Cu") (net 5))
 (segment (start 125.476 107.188) (end 124.175 105.887) (width 0.3) (layer "B.Cu") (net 5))
 (segment (start 118.11 120.65) (end 123.19 125.73) (width 0.3) (layer "B.Cu") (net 5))
 (segment (start 123.19 125.73) (end 123.19 125.984) (width 0.3) (layer "B.Cu") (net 5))
 (segment (start 118.11 108.712) (end 118.11 120.65) (width 0.3) (layer "B.Cu") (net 5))
 (segment (start 124.175 105.887) (end 120.935 105.887) (width 0.3) (layer "B.Cu") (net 5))
 (segment (start 120.935 105.887) (end 118.11 108.712) (width 0.3) (layer "B.Cu") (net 5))
 (segment (start 120.150818 134.874) (end 125.222 134.874) (width 0.3) (layer "F.Cu") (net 7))
 (segment (start 119.634 107.188) (end 118.11 108.712) (width 0.3) (layer "F.Cu") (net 7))
 (segment (start 118.11 108.712) (end 118.11 132.833182) (width 0.3) (layer "F.Cu") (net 7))
 (segment (start 125.222 134.874) (end 130.81 129.286) (width 0.3) (layer "F.Cu") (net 7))
 (segment (start 130.81 129.032) (end 130.556 128.778) (width 0.3) (layer "F.Cu") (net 7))
 (segment (start 118.11 132.833182) (end 120.150818 134.874) (width 0.3) (layer "F.Cu") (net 7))
 (segment (start 122.936 107.188) (end 119.634 107.188) (width 0.3) (layer "F.Cu") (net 7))
 (segment (start 130.81 129.286) (end 130.81 129.032) (width 0.3) (layer "F.Cu") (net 7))
 (segment (start 124.949 124.949) (end 123.698 123.698) (width 0.3) (layer "F.Cu") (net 14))
 (segment (start 123.698 123.698) (end 122.936 123.698) (width 0.3) (layer "F.Cu") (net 14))
 (segment (start 132.099 124.949) (end 124.949 124.949) (width 0.3) (layer "F.Cu") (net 14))
 (segment (start 135.89 121.158) (end 132.099 124.949) (width 0.3) (layer "F.Cu") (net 14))
 (via (at 135.89 121.158) (size 0.7) (drill 0.5) (layers "F.Cu" "B.Cu") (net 14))
 (segment (start 139.954 121.158) (end 141.906 123.11) (width 0.3) (layer "B.Cu") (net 14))
 (segment (start 135.89 121.158) (end 139.954 121.158) (width 0.3) (layer "B.Cu") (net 14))
 (segment (start 140.462 128.611958) (end 140.462 133.858) (width 0.3) (layer "F.Cu") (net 9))
 (segment (start 135.53 123.679958) (end 140.462 128.611958) (width 0.3) (layer "F.Cu") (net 9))
 (segment (start 136.336042 121.734) (end 135.53 122.540042) (width 0.3) (layer "F.Cu") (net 9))
 (segment (start 130.992 114.714) (end 137.475958 121.197958) (width 0.3) (layer "F.Cu") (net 9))
 (segment (start 135.53 122.540042) (end 135.53 123.679958) (width 0.3) (layer "F.Cu") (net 9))
 (segment (start 126.84 114.714) (end 130.992 114.714) (width 0.3) (layer "F.Cu") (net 9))
 (segment (start 137.475958 121.734) (end 136.336042 121.734) (width 0.3) (layer "F.Cu") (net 9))
 (segment (start 122.936 118.618) (end 126.84 114.714) (width 0.3) (layer "F.Cu") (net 9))
 (segment (start 137.475958 121.197958) (end 137.475958 121.734) (width 0.3) (layer "F.Cu") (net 9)))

